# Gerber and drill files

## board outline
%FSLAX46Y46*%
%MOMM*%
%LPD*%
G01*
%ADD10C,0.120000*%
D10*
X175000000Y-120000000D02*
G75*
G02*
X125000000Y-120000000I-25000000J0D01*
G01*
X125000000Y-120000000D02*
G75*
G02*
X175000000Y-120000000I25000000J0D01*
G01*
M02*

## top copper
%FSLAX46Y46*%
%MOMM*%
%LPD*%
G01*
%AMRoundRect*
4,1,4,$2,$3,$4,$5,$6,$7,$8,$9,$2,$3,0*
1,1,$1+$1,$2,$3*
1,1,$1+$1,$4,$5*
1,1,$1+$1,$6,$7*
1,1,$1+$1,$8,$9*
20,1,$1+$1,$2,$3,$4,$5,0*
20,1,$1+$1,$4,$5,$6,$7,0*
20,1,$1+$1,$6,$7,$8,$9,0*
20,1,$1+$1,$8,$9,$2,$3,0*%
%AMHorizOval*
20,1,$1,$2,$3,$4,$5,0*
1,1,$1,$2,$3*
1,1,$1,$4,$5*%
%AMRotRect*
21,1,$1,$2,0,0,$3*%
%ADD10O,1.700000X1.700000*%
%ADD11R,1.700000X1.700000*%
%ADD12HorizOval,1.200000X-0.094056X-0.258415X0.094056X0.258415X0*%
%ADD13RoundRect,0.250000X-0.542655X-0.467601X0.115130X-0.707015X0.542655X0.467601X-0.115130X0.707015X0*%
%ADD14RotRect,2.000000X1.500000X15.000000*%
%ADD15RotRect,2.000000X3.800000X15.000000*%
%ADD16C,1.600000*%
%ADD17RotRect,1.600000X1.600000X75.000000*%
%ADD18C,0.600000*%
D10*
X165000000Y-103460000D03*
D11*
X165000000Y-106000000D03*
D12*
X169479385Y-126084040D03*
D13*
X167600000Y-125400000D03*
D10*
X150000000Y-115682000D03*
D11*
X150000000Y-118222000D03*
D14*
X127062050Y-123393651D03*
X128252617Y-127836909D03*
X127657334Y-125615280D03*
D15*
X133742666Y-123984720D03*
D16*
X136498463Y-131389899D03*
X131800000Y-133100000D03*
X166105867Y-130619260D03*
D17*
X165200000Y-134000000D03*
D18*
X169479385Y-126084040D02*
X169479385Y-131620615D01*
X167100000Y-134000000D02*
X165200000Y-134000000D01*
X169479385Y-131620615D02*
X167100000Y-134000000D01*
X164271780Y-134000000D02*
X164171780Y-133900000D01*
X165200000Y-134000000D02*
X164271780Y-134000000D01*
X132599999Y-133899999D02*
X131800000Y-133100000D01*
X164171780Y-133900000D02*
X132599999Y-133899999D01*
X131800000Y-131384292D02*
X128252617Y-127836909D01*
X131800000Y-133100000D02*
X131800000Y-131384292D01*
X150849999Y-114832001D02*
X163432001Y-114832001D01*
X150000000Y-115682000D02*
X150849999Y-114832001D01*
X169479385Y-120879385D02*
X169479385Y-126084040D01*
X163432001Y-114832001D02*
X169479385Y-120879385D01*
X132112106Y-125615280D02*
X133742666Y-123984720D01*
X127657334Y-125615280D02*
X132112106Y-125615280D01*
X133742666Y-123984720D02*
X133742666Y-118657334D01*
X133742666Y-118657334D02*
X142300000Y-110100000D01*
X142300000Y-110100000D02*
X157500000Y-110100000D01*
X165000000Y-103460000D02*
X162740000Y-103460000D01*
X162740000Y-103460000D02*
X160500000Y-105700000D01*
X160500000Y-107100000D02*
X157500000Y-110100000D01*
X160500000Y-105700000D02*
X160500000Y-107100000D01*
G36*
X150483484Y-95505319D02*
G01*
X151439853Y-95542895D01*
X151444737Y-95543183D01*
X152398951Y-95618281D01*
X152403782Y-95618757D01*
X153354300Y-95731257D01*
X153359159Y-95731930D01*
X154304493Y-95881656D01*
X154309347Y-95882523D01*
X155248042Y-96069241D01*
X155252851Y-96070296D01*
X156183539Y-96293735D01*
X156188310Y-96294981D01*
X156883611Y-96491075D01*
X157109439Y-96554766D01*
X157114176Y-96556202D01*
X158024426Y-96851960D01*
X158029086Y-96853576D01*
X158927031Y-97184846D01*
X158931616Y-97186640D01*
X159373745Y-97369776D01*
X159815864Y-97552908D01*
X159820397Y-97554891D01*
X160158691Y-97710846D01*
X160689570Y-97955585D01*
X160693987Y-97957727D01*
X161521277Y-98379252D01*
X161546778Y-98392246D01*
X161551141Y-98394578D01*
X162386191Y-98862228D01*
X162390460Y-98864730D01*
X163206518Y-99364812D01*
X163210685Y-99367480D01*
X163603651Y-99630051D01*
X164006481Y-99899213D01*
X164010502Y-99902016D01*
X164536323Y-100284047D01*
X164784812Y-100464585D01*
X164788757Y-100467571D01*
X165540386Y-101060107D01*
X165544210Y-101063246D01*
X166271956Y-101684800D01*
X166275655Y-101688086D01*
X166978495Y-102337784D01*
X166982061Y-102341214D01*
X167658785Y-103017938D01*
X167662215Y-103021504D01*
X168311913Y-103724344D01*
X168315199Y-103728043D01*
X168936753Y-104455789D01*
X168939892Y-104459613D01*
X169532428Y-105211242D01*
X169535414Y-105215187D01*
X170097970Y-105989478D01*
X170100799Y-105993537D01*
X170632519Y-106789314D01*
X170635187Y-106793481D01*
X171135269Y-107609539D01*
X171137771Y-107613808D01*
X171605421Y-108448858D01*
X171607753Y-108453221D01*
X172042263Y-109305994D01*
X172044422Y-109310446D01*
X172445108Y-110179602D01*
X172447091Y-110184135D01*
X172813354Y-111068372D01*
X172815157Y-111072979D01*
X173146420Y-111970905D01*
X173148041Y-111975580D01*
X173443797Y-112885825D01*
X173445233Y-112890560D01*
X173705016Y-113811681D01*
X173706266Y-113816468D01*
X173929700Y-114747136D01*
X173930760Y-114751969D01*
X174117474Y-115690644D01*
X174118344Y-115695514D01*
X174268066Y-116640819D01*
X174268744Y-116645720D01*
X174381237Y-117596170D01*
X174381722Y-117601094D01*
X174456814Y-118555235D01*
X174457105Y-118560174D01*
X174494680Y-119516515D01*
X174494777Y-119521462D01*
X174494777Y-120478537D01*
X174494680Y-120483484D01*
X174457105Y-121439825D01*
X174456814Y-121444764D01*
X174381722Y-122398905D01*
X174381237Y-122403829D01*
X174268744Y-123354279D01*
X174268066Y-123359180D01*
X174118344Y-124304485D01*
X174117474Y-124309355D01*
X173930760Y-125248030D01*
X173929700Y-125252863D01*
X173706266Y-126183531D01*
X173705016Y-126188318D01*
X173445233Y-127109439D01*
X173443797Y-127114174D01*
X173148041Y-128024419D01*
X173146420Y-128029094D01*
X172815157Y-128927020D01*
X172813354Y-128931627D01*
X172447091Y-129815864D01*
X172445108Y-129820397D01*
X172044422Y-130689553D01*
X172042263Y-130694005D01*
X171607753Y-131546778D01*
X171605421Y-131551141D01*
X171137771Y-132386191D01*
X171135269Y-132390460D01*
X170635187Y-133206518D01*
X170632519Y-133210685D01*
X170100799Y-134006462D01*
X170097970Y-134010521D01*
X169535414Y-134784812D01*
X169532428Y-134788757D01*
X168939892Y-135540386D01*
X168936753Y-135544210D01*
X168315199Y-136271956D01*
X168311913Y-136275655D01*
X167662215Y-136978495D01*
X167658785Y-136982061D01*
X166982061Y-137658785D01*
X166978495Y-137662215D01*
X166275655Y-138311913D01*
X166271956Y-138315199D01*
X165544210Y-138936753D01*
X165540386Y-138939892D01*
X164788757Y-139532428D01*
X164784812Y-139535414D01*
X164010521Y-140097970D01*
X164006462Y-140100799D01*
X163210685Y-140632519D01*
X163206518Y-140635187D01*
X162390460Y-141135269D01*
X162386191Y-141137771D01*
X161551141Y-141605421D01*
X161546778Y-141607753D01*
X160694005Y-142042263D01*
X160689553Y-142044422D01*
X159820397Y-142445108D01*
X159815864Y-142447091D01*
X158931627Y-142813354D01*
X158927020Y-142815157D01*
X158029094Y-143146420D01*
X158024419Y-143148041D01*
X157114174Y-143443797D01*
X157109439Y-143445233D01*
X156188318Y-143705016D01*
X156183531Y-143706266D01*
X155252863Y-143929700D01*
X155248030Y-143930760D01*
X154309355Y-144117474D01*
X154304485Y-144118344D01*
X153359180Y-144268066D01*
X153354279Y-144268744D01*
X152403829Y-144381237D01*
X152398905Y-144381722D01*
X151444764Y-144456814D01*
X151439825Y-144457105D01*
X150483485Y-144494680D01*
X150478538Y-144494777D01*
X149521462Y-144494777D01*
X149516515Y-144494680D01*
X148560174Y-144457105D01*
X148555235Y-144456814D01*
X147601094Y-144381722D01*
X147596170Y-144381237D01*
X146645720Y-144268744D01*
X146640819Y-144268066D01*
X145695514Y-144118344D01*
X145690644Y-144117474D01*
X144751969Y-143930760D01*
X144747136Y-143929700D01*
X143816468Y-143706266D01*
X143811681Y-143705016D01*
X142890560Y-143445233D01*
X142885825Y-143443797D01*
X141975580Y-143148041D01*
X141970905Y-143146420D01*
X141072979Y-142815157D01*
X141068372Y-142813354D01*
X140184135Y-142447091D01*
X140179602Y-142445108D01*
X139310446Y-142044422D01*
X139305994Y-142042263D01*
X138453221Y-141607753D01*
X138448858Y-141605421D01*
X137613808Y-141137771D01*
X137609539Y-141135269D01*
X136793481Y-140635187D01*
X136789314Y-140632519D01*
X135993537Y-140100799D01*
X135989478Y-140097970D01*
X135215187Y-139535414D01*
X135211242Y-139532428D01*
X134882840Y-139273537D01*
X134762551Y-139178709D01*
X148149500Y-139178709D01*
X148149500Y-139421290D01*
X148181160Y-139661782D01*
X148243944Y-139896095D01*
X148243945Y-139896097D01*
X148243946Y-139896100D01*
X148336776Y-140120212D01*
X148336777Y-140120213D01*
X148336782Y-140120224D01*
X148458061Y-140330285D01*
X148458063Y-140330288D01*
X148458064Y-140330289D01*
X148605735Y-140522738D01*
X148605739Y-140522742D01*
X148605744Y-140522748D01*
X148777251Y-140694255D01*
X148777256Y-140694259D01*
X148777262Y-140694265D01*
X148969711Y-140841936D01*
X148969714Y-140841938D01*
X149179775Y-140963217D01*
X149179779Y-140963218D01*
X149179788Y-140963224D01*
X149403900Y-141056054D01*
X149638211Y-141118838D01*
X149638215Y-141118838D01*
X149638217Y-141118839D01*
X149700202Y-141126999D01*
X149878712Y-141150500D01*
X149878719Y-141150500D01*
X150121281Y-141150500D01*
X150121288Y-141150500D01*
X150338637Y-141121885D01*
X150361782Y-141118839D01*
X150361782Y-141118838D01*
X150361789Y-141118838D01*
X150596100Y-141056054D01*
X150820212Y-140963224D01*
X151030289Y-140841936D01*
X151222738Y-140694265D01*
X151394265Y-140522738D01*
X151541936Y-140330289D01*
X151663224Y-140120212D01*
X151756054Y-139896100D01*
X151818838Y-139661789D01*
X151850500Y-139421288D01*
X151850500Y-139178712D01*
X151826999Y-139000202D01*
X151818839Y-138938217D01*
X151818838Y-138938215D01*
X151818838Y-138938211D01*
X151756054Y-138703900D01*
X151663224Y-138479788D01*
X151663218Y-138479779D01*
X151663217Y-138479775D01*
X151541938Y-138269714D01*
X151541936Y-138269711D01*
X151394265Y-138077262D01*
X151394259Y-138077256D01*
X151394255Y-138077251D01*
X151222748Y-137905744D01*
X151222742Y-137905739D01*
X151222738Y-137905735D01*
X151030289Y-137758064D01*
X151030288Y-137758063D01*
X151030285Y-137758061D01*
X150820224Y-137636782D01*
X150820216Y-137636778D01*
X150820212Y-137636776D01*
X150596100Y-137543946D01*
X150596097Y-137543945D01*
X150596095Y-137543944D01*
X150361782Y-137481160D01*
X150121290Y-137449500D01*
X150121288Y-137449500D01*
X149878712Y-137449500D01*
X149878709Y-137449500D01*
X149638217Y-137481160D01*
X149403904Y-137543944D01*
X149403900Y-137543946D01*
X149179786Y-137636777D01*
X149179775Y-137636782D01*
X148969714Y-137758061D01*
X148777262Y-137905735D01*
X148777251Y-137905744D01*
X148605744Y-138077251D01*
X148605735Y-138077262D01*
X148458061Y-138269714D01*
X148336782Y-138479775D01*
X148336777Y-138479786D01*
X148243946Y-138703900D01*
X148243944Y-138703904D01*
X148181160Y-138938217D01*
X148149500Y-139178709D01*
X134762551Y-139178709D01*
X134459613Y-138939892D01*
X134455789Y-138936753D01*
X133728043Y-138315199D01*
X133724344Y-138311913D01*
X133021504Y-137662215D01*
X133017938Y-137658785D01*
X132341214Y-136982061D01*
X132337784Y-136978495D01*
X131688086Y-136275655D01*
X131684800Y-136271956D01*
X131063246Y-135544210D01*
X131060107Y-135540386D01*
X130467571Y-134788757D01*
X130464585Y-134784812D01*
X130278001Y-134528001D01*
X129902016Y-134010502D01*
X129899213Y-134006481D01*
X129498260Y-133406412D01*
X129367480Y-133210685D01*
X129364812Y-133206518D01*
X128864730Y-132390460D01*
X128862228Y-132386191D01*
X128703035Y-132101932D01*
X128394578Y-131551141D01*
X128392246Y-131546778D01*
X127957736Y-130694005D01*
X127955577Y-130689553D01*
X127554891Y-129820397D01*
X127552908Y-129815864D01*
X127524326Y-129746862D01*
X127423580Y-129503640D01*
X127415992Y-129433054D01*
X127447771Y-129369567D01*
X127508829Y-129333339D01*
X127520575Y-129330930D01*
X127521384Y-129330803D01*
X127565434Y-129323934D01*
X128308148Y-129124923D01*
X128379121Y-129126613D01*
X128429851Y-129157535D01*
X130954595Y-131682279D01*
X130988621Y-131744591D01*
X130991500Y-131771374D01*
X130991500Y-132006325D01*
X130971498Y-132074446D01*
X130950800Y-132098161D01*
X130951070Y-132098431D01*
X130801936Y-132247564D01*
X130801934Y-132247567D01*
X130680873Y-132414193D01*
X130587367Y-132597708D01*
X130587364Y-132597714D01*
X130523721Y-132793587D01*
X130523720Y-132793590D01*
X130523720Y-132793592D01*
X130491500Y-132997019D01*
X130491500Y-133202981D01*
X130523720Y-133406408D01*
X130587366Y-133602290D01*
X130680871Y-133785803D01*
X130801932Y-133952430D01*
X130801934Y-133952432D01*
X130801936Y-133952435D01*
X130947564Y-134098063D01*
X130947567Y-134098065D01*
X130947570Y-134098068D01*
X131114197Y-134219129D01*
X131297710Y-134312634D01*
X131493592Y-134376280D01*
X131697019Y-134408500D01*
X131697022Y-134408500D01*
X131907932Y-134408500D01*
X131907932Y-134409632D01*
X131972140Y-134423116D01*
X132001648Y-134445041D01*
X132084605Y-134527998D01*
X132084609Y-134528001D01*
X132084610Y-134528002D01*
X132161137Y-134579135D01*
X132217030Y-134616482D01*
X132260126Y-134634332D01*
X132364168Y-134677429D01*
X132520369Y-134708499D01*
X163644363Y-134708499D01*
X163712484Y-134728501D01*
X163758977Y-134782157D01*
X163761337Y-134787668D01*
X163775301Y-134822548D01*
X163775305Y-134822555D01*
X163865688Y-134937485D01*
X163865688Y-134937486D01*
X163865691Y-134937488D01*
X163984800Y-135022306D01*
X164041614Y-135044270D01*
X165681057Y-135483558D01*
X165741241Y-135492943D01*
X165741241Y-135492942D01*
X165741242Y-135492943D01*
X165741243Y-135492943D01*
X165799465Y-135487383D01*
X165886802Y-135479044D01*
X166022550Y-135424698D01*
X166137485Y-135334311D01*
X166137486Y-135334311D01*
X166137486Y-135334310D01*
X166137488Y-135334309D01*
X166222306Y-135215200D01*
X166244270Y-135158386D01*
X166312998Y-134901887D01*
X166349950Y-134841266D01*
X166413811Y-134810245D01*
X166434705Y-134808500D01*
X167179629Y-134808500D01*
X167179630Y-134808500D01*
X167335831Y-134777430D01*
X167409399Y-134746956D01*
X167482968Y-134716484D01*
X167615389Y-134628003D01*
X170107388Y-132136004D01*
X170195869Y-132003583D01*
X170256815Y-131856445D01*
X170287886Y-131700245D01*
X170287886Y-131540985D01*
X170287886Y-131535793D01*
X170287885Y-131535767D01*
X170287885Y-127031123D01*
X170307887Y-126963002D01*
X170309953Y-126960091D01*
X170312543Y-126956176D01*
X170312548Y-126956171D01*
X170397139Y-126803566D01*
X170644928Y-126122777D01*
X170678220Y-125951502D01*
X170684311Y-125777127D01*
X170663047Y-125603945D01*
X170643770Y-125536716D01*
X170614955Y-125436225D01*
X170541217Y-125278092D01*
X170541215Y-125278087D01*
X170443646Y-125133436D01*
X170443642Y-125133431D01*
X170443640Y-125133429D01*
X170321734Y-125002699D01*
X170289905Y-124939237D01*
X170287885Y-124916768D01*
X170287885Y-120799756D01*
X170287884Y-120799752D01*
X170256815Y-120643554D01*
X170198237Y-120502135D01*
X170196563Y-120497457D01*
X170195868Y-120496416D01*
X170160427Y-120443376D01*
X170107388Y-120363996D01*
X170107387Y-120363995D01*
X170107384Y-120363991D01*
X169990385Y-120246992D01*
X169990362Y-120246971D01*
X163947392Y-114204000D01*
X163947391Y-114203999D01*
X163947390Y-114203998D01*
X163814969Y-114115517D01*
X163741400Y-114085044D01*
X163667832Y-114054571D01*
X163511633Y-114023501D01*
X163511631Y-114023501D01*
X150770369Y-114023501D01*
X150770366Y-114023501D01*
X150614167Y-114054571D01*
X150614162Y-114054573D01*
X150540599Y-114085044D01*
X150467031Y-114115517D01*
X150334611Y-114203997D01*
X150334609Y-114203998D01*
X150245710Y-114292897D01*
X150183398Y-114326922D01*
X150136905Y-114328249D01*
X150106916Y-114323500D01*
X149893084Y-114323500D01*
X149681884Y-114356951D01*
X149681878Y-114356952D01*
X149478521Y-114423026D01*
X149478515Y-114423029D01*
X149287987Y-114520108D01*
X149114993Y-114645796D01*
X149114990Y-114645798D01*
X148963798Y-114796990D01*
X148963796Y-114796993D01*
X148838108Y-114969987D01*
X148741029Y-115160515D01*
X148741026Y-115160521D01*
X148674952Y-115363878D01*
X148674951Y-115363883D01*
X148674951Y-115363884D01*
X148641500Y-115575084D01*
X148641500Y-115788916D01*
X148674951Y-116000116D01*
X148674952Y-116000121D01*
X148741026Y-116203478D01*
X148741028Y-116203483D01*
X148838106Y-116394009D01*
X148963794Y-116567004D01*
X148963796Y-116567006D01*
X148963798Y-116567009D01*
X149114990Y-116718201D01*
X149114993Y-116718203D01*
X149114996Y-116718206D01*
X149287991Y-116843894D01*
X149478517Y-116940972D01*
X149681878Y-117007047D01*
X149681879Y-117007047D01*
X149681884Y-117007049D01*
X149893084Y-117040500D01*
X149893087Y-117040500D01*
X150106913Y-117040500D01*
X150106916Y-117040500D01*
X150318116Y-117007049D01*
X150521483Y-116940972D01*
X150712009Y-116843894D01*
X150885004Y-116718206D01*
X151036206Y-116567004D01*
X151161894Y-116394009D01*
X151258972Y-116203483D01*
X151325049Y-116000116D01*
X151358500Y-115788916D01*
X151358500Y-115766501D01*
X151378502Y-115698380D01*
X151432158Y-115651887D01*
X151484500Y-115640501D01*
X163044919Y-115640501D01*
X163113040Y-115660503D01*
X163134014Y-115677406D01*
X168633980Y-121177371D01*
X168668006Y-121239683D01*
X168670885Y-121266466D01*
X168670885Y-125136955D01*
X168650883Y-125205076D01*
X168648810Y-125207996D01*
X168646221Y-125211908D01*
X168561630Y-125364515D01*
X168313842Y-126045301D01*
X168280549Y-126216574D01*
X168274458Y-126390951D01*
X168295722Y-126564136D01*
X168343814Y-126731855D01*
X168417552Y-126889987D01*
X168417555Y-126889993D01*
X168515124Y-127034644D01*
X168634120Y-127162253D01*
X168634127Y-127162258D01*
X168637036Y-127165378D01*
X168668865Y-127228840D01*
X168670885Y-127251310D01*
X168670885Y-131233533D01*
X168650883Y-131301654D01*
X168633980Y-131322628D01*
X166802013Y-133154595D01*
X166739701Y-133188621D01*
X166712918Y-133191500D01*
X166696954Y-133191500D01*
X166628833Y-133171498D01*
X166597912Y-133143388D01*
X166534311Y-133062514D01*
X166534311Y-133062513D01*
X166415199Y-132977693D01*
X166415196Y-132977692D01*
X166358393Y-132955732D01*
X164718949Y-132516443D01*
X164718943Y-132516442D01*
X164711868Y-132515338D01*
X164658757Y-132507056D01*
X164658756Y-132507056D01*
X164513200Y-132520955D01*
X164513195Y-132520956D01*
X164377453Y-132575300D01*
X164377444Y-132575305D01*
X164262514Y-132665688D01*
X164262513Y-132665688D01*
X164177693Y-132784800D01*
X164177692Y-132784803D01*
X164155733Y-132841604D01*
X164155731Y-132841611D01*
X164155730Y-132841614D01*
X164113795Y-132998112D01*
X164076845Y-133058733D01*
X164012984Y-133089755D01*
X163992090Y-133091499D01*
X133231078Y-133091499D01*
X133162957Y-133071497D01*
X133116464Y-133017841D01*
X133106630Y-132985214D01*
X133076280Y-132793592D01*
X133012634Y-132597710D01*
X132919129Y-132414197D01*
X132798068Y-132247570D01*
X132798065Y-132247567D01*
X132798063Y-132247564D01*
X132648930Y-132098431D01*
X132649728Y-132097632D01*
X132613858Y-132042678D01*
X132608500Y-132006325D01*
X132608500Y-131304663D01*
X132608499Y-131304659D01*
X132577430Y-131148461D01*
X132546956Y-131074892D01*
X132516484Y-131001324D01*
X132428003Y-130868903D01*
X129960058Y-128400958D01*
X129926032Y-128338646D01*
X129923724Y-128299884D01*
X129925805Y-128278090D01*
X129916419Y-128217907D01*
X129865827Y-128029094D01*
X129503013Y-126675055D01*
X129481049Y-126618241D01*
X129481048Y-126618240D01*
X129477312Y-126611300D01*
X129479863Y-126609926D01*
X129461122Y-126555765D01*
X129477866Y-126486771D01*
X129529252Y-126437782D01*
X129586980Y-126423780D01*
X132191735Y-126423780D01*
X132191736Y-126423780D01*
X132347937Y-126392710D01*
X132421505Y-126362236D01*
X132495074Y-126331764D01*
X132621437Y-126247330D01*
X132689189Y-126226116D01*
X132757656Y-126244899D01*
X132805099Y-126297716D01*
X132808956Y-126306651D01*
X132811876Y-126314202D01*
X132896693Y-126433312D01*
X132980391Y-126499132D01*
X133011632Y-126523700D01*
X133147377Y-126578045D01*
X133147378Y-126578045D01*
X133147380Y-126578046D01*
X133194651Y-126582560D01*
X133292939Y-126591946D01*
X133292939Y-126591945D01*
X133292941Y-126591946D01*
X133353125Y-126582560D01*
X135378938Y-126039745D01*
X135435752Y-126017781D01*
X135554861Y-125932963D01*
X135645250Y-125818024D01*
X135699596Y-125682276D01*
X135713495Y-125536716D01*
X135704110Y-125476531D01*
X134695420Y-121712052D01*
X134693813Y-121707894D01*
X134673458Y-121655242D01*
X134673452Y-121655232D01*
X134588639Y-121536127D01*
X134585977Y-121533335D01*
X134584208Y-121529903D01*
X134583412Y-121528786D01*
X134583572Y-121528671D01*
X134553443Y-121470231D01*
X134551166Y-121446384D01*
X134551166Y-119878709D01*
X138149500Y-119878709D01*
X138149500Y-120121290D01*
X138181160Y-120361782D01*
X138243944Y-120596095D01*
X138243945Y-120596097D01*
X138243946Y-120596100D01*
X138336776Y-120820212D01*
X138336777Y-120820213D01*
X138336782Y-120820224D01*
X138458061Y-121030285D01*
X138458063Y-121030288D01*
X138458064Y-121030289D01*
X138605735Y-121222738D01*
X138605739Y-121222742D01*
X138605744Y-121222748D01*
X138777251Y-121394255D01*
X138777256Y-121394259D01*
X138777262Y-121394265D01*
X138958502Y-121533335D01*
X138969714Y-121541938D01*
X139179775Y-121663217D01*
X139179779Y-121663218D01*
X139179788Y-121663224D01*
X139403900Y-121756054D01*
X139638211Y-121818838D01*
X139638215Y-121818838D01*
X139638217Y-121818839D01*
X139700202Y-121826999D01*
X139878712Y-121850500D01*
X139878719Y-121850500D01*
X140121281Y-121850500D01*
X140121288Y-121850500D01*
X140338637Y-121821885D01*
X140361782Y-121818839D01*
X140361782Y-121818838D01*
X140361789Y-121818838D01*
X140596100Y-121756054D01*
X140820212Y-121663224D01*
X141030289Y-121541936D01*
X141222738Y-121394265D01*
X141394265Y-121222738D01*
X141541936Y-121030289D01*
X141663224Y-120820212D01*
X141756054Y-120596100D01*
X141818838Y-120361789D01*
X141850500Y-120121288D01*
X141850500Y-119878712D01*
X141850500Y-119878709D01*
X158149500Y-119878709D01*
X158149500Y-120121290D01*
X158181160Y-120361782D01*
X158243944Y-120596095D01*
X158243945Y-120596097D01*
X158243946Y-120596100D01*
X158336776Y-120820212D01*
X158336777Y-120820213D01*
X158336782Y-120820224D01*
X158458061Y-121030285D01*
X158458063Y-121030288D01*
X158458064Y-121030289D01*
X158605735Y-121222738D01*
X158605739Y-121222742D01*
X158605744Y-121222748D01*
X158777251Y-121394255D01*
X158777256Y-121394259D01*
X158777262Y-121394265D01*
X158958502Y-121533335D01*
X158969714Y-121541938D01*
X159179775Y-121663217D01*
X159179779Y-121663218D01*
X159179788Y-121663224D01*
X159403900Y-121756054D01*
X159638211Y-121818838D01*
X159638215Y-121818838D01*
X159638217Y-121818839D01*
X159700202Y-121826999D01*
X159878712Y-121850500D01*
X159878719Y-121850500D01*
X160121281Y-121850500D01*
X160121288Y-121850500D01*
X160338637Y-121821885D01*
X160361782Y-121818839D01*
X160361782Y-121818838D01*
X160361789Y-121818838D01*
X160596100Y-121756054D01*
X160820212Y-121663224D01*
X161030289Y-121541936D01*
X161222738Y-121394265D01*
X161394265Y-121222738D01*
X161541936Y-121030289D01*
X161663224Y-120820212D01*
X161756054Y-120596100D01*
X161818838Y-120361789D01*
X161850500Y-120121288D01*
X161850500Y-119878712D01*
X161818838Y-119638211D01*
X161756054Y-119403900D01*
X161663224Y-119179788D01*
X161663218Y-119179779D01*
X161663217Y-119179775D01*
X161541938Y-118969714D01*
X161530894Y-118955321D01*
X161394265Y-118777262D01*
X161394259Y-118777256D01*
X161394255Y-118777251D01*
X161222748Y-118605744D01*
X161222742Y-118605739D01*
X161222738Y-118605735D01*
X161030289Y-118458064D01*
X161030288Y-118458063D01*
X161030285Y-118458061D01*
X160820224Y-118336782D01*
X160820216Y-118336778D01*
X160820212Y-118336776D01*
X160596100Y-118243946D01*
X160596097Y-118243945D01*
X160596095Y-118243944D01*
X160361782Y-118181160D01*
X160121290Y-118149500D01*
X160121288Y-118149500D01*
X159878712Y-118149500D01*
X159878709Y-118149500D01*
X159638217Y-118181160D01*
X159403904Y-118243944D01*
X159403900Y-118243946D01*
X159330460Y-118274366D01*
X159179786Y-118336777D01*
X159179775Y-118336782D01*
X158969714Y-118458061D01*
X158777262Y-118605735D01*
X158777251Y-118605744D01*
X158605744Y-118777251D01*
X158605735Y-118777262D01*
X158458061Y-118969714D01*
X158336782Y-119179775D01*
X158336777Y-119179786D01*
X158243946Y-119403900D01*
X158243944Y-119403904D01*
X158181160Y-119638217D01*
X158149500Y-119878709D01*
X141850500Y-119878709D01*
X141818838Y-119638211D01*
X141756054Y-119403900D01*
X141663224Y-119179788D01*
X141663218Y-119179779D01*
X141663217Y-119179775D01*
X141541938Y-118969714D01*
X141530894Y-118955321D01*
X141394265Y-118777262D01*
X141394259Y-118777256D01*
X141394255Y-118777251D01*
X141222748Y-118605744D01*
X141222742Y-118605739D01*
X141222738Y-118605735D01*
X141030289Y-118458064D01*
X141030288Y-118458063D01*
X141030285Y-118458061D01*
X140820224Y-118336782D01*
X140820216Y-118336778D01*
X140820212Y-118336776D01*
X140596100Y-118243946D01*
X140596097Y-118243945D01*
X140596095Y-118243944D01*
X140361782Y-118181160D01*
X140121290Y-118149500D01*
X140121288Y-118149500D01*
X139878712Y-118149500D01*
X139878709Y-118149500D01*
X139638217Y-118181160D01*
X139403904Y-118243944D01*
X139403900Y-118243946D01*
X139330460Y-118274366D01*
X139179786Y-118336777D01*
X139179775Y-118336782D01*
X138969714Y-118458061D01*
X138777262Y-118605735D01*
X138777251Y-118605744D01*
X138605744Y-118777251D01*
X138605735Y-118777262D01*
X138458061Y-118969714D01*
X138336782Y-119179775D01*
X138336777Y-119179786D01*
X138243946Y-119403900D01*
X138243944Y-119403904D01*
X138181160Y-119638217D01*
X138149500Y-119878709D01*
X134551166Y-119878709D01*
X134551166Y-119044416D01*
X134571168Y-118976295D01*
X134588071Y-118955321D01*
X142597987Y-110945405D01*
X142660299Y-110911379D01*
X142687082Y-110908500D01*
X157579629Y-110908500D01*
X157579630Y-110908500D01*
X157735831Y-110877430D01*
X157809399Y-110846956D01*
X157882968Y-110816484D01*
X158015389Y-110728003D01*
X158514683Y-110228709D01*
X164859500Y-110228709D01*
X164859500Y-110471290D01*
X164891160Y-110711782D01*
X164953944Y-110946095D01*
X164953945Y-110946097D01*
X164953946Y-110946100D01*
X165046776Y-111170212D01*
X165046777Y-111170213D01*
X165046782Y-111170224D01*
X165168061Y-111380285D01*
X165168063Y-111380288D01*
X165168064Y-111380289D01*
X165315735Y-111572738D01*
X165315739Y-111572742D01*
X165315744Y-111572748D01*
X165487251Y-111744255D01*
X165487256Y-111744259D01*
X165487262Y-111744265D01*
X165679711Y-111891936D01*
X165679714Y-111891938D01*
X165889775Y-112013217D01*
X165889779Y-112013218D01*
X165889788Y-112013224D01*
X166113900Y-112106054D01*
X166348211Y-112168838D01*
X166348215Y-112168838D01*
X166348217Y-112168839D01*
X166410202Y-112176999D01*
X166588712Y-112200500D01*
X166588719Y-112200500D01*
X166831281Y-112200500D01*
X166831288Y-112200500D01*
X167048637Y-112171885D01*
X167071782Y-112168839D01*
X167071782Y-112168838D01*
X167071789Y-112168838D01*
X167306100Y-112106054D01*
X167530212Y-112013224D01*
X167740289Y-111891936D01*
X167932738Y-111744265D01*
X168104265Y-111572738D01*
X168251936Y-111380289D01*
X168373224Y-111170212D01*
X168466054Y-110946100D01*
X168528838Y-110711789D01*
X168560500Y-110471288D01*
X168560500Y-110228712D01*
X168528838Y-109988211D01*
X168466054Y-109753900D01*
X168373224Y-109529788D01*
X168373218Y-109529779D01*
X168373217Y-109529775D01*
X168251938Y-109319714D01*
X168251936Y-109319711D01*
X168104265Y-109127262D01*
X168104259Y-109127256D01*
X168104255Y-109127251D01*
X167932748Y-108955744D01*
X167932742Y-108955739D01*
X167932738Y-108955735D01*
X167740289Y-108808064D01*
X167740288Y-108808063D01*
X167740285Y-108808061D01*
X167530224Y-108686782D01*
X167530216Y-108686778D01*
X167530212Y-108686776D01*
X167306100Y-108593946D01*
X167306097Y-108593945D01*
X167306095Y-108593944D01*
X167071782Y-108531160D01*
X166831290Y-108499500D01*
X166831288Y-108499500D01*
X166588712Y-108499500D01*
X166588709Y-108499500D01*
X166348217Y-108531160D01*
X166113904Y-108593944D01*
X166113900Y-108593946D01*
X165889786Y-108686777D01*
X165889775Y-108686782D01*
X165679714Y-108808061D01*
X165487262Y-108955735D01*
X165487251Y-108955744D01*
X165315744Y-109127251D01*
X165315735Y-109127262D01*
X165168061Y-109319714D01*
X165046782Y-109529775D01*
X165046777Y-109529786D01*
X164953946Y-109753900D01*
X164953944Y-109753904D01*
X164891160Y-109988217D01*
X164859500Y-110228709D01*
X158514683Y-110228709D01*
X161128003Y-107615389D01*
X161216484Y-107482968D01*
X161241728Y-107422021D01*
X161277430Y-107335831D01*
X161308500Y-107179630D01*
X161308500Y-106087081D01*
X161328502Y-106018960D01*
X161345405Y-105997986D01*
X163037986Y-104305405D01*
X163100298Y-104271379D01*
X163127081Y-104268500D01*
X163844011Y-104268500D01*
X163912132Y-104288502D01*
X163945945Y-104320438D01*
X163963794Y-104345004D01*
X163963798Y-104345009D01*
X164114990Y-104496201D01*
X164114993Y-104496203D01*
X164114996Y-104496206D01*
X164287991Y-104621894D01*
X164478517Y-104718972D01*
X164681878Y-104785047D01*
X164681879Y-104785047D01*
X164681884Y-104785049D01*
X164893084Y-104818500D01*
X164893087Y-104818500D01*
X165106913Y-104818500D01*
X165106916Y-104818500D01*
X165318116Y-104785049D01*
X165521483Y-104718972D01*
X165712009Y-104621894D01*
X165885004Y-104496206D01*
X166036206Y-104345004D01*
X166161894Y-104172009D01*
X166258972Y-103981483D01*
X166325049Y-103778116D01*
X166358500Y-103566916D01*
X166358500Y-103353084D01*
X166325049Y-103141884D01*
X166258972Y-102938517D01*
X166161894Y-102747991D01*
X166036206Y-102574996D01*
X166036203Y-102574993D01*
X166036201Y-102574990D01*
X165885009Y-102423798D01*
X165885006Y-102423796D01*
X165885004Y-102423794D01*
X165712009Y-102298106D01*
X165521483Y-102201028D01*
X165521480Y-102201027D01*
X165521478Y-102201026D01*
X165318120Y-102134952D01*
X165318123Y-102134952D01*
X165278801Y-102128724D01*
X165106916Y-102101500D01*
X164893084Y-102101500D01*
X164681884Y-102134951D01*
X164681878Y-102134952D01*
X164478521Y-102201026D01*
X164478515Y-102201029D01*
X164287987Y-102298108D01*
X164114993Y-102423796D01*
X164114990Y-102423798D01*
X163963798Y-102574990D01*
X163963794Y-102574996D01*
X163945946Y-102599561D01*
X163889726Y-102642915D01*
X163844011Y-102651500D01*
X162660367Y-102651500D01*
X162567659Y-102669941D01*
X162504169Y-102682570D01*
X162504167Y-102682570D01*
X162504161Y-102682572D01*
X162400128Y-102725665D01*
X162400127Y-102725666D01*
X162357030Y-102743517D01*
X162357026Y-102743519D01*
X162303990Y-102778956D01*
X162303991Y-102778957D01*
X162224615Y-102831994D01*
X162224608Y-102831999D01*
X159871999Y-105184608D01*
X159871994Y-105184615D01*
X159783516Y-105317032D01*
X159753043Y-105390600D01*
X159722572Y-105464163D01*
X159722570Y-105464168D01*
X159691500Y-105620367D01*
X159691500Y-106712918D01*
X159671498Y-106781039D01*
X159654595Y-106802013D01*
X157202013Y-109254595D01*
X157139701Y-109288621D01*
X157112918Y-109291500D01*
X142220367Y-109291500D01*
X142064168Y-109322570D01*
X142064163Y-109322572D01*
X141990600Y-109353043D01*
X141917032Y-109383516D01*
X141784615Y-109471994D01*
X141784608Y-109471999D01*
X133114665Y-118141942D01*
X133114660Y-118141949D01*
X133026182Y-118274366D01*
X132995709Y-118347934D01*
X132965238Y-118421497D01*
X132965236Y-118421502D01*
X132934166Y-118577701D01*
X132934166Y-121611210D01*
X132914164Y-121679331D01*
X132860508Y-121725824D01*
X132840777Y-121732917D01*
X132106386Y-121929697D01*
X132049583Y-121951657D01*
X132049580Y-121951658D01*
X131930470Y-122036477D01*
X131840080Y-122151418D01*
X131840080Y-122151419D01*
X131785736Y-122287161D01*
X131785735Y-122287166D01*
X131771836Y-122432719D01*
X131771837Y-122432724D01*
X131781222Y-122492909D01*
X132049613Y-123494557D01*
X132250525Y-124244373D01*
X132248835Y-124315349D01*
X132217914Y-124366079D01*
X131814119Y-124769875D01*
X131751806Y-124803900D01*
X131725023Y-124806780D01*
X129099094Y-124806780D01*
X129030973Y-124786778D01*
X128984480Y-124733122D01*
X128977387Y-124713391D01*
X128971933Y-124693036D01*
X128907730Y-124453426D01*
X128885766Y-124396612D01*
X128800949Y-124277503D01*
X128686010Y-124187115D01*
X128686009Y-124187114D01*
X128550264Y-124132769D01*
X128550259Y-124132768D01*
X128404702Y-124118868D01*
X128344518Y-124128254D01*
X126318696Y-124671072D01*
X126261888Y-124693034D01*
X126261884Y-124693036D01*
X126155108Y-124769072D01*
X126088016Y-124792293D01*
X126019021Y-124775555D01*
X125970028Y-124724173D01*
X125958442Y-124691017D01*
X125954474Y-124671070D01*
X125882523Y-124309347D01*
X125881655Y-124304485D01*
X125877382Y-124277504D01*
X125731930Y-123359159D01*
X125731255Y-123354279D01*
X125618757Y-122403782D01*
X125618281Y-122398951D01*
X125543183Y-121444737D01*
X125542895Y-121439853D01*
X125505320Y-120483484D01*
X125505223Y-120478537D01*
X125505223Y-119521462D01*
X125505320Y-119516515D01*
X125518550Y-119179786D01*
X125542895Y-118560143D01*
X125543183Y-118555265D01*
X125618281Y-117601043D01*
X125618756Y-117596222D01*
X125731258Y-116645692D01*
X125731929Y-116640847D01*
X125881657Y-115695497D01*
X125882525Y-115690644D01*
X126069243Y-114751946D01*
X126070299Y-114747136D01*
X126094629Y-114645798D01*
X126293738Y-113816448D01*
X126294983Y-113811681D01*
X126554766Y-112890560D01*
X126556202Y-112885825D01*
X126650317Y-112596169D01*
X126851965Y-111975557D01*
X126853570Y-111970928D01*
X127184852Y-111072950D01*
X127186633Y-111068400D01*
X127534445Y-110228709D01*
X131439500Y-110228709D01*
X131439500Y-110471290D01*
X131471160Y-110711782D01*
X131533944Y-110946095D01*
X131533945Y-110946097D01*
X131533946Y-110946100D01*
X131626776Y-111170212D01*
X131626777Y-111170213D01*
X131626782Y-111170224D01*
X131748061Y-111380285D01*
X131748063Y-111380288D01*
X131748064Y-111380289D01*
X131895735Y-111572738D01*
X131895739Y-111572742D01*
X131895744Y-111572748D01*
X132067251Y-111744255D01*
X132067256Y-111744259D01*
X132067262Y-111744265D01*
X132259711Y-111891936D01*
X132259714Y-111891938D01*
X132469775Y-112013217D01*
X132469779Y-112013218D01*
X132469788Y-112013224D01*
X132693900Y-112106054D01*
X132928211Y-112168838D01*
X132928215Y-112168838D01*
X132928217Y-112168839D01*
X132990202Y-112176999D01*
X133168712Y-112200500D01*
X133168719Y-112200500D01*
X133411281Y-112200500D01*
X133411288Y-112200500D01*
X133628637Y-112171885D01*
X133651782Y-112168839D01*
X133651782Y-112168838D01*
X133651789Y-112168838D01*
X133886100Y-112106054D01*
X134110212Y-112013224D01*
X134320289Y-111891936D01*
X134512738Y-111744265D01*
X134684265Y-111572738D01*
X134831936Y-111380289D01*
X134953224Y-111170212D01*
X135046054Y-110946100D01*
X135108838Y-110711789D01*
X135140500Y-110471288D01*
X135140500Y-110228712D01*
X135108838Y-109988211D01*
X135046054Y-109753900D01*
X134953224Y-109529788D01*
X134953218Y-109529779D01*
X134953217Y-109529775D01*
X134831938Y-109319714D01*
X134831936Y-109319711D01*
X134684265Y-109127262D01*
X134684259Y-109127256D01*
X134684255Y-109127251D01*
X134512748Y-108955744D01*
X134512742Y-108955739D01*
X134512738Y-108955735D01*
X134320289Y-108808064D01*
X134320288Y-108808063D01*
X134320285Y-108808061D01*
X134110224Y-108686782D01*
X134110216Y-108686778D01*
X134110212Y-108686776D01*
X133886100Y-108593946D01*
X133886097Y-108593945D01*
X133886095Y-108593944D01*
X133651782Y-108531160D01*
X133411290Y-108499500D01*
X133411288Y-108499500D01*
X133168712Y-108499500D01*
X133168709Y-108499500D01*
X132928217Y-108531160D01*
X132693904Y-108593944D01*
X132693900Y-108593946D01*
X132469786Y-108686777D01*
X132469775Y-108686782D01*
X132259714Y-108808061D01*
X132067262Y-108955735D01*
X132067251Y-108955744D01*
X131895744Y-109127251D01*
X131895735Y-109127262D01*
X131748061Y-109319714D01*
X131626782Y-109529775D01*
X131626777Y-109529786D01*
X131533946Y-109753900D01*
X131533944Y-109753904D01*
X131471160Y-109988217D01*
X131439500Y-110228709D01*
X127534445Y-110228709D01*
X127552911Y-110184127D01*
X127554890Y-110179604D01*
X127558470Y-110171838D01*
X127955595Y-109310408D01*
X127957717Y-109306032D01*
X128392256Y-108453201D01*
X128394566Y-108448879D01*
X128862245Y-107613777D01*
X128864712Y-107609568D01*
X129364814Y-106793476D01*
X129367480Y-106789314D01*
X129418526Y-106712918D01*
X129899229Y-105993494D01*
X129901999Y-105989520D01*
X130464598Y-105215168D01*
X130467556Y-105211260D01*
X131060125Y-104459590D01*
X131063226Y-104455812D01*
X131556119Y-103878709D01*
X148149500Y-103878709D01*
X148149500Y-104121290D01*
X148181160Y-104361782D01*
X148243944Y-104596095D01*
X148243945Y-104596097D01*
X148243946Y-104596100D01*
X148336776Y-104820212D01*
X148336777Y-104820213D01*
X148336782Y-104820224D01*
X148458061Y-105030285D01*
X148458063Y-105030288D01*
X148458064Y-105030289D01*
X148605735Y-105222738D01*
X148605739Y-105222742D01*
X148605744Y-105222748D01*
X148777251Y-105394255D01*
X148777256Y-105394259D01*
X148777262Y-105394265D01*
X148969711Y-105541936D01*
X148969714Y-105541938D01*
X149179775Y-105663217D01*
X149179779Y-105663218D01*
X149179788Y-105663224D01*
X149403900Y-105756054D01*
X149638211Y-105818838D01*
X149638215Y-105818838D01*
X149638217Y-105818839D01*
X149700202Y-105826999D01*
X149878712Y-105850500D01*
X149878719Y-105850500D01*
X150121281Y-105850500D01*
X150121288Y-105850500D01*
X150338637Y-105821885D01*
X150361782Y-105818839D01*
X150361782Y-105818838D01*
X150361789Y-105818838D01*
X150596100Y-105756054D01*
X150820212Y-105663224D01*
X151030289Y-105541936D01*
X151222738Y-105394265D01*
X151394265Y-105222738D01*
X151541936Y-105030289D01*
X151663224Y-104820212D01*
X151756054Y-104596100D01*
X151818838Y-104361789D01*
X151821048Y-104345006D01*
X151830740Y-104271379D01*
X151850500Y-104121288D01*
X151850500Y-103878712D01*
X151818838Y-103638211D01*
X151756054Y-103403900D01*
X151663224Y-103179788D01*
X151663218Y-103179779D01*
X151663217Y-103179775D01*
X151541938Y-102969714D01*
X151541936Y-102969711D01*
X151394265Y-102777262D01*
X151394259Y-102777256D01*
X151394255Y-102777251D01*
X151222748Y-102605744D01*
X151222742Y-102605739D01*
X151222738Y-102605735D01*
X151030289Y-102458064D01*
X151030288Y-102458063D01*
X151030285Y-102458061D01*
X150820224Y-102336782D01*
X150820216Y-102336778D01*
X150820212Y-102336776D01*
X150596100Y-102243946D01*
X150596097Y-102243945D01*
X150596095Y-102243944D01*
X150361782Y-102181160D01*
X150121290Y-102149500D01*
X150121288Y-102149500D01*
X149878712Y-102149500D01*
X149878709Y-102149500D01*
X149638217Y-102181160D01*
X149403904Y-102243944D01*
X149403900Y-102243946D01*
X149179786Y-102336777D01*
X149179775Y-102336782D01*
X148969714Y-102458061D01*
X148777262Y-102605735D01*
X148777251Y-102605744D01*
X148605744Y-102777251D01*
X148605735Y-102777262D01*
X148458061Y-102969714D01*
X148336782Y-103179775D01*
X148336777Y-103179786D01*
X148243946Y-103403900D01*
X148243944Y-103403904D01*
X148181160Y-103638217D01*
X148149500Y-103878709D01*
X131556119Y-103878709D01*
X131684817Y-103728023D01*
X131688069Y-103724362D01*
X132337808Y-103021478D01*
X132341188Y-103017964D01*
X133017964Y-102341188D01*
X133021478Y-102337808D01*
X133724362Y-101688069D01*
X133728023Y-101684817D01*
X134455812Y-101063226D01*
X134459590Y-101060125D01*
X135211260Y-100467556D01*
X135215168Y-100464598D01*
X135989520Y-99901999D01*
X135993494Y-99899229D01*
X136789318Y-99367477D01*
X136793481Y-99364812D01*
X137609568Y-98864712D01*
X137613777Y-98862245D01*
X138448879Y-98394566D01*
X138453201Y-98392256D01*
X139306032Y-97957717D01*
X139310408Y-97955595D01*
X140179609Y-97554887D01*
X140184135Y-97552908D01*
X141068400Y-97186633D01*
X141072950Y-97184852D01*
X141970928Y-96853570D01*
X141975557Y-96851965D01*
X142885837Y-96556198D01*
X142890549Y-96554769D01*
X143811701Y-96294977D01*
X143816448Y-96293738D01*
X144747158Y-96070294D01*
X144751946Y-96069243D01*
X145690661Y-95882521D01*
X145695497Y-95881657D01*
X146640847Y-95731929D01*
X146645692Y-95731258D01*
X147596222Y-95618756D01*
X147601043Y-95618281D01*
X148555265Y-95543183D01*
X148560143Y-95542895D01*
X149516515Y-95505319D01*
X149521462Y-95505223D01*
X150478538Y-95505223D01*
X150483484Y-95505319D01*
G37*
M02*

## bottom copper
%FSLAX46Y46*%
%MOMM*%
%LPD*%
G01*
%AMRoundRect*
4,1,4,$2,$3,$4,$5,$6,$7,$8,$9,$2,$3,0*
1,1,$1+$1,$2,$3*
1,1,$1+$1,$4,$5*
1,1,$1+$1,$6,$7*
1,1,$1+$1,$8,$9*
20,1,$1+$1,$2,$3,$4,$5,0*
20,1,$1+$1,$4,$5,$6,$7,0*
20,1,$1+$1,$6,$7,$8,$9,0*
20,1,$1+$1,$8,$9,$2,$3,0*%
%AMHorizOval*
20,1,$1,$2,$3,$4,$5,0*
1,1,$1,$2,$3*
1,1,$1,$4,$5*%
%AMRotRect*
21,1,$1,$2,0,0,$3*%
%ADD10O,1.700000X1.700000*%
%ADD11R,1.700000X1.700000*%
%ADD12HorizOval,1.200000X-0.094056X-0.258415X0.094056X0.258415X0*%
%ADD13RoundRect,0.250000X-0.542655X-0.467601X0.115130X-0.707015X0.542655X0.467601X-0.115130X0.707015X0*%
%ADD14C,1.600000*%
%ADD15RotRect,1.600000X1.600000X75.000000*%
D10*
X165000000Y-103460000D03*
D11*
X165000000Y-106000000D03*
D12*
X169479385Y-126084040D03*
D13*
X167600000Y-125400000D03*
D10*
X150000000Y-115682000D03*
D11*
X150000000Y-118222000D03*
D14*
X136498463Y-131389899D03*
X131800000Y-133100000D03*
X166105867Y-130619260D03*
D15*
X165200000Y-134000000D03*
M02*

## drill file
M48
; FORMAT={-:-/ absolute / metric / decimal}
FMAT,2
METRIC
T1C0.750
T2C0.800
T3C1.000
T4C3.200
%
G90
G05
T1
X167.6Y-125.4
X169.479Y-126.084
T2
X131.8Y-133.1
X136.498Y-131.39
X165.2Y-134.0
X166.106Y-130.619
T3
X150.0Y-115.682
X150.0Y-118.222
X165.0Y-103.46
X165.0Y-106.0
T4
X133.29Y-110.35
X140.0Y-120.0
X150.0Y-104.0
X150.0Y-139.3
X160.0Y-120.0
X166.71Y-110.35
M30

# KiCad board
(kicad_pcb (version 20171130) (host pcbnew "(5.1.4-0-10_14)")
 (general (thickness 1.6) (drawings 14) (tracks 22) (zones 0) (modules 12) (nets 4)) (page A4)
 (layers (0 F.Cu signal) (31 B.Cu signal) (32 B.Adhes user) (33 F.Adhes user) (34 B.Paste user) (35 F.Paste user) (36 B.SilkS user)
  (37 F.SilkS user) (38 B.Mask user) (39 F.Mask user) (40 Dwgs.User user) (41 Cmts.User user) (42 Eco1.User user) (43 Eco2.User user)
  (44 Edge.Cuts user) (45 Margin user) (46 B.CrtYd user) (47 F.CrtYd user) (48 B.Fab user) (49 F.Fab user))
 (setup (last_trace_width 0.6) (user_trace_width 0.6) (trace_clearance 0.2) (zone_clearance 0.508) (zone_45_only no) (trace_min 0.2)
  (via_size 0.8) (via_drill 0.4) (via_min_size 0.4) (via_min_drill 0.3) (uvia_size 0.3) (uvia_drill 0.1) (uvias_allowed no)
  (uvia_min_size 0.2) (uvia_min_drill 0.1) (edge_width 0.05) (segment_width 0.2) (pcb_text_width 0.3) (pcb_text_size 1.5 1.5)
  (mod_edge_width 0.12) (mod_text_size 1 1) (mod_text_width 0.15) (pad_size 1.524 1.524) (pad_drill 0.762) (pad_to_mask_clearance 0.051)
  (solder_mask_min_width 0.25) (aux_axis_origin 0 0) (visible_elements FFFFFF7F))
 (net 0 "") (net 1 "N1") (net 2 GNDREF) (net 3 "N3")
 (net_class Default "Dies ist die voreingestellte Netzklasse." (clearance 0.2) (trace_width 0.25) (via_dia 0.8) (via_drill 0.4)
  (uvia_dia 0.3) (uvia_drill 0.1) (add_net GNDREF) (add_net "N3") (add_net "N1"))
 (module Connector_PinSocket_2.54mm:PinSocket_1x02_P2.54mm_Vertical (layer B.Cu) (at 165 106)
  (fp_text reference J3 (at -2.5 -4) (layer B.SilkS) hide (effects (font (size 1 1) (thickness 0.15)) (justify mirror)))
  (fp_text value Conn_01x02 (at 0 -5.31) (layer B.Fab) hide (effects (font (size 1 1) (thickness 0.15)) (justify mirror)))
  (pad 2 thru_hole oval (at 0 -2.54) (size 1.7 1.7) (drill 1) (layers *.Cu *.Mask) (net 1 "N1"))
  (pad 1 thru_hole rect (at 0 0) (size 1.7 1.7) (drill 1) (layers *.Cu *.Mask) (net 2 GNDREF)))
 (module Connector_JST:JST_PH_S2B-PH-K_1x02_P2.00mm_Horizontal (layer B.Cu) (at 167.6 125.4 340)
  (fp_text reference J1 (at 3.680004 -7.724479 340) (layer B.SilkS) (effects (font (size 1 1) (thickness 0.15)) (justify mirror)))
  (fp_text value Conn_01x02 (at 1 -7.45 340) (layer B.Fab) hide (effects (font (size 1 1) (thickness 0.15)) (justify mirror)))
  (pad 2 thru_hole oval (at 2 0 340) (size 1.2 1.75) (drill 0.75) (layers *.Cu *.Mask) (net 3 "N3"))
  (pad 1 thru_hole roundrect (at 0 0 340) (size 1.2 1.75) (drill 0.75) (layers *.Cu *.Mask) (roundrect_rratio 0.208333) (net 2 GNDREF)))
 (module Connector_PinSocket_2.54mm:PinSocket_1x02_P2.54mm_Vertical (layer F.Cu) (at 150 118.222 180)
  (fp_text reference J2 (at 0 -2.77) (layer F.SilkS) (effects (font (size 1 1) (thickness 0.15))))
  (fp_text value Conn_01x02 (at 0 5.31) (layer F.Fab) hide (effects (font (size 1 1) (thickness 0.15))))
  (pad 2 thru_hole oval (at 0 2.54 180) (size 1.7 1.7) (drill 1) (layers *.Cu *.Mask) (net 3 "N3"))
  (pad 1 thru_hole rect (at 0 0 180) (size 1.7 1.7) (drill 1) (layers *.Cu *.Mask) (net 2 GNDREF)))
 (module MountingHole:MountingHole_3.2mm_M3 (layer F.Cu) (at 160 120)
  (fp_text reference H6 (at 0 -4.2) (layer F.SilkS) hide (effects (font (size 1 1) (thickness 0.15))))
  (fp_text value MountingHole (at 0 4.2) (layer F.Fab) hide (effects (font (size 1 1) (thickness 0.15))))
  (pad 1 np_thru_hole circle (at 0 0) (size 3.2 3.2) (drill 3.2) (layers *.Cu *.Mask)))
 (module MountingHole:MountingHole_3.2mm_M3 (layer F.Cu) (at 140 120)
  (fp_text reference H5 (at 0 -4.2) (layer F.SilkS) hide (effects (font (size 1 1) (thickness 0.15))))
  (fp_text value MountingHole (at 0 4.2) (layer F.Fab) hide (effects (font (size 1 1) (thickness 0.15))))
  (pad 1 np_thru_hole circle (at 0 0) (size 3.2 3.2) (drill 3.2) (layers *.Cu *.Mask)))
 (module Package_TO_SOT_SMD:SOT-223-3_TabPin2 (layer F.Cu) (at 130.7 124.8 15)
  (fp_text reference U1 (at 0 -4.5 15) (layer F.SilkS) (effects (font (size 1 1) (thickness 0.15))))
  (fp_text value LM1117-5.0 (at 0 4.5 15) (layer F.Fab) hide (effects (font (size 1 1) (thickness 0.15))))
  (pad 1 smd rect (at -3.15 -2.3 15) (size 2 1.5) (layers F.Cu F.Paste F.Mask) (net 2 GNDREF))
  (pad 3 smd rect (at -3.15 2.3 15) (size 2 1.5) (layers F.Cu F.Paste F.Mask) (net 3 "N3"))
  (pad 2 smd rect (at -3.15 0 15) (size 2 1.5) (layers F.Cu F.Paste F.Mask) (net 1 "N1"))
  (pad 2 smd rect (at 3.15 0 15) (size 2 3.8) (layers F.Cu F.Paste F.Mask) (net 1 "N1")))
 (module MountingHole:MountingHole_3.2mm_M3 (layer F.Cu) (at 133.29 110.35)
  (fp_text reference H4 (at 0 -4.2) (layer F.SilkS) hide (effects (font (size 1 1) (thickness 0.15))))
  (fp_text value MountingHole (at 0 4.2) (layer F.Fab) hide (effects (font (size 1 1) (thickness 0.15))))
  (pad 1 np_thru_hole circle (at 0 0) (size 3.2 3.2) (drill 3.2) (layers *.Cu *.Mask)))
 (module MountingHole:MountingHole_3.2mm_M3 (layer F.Cu) (at 166.71 110.35)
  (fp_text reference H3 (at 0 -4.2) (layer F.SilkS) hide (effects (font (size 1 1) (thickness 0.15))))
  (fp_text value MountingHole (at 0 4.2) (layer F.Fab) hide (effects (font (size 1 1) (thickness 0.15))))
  (pad 1 np_thru_hole circle (at 0 0) (size 3.2 3.2) (drill 3.2) (layers *.Cu *.Mask)))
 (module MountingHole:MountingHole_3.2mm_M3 (layer F.Cu) (at 150 139.3)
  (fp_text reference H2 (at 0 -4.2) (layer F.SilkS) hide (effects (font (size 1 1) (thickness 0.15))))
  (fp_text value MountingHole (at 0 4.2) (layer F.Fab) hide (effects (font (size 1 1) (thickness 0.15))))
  (pad 1 np_thru_hole circle (at 0 0) (size 3.2 3.2) (drill 3.2) (layers *.Cu *.Mask)))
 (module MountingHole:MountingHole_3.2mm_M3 (layer F.Cu) (at 150 104)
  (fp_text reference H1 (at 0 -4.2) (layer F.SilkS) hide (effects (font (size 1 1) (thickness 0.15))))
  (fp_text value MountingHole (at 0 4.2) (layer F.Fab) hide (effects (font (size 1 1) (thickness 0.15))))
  (pad 1 np_thru_hole circle (at 0 0) (size 3.2 3.2) (drill 3.2) (layers *.Cu *.Mask)))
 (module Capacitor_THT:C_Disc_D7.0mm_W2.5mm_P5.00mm (layer F.Cu) (at 131.8 133.1 20)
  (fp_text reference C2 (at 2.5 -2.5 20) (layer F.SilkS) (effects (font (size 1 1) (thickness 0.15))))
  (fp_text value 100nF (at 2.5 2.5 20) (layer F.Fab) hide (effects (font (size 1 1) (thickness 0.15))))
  (pad 2 thru_hole circle (at 5 0 20) (size 1.6 1.6) (drill 0.8) (layers *.Cu *.Mask) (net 2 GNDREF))
  (pad 1 thru_hole circle (at 0 0 20) (size 1.6 1.6) (drill 0.8) (layers *.Cu *.Mask) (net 3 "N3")))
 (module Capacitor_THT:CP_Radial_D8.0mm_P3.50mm (layer F.Cu) (at 165.2 134 75)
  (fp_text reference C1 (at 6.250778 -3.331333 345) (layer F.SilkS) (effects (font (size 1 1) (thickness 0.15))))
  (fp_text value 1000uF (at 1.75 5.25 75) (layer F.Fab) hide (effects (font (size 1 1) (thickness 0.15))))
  (pad 2 thru_hole circle (at 3.5 0 75) (size 1.6 1.6) (drill 0.8) (layers *.Cu *.Mask) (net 2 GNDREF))
  (pad 1 thru_hole rect (at 0 0 75) (size 1.6 1.6) (drill 0.8) (layers *.Cu *.Mask) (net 3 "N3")))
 (gr_circle (center 150 120) (end 175 120) (layer Edge.Cuts) (width 0.12))
 (segment (start 169.479385 126.08404) (end 169.479385 131.620615) (width 0.6) (layer F.Cu) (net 3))
 (segment (start 167.1 134) (end 165.2 134) (width 0.6) (layer F.Cu) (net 3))
 (segment (start 169.479385 131.620615) (end 167.1 134) (width 0.6) (layer F.Cu) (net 3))
 (segment (start 164.27178 134) (end 164.17178 133.9) (width 0.6) (layer F.Cu) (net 3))
 (segment (start 165.2 134) (end 164.27178 134) (width 0.6) (layer F.Cu) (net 3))
 (segment (start 132.599999 133.899999) (end 131.8 133.1) (width 0.6) (layer F.Cu) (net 3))
 (segment (start 164.17178 133.9) (end 132.599999 133.899999) (width 0.6) (layer F.Cu) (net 3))
 (segment (start 131.8 131.384292) (end 128.252617 127.836909) (width 0.6) (layer F.Cu) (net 3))
 (segment (start 131.8 133.1) (end 131.8 131.384292) (width 0.6) (layer F.Cu) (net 3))
 (segment (start 150.849999 114.832001) (end 163.432001 114.832001) (width 0.6) (layer F.Cu) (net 3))
 (segment (start 150 115.682) (end 150.849999 114.832001) (width 0.6) (layer F.Cu) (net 3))
 (segment (start 169.479385 120.879385) (end 169.479385 126.08404) (width 0.6) (layer F.Cu) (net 3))
 (segment (start 163.432001 114.832001) (end 169.479385 120.879385) (width 0.6) (layer F.Cu) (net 3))
 (segment (start 132.112106 125.61528) (end 133.742666 123.98472) (width 0.6) (layer F.Cu) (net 1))
 (segment (start 127.657334 125.61528) (end 132.112106 125.61528) (width 0.6) (layer F.Cu) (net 1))
 (segment (start 133.742666 123.98472) (end 133.742666 118.657334) (width 0.6) (layer F.Cu) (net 1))
 (segment (start 133.742666 118.657334) (end 142.3 110.1) (width 0.6) (layer F.Cu) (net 1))
 (segment (start 142.3 110.1) (end 157.5 110.1) (width 0.6) (layer F.Cu) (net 1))
 (segment (start 165 103.46) (end 162.74 103.46) (width 0.6) (layer F.Cu) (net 1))
 (segment (start 162.74 103.46) (end 160.5 105.7) (width 0.6) (layer F.Cu) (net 1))
 (segment (start 160.5 107.1) (end 157.5 110.1) (width 0.6) (layer F.Cu) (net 1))
 (segment (start 160.5 105.7) (end 160.5 107.1) (width 0.6) (layer F.Cu) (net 1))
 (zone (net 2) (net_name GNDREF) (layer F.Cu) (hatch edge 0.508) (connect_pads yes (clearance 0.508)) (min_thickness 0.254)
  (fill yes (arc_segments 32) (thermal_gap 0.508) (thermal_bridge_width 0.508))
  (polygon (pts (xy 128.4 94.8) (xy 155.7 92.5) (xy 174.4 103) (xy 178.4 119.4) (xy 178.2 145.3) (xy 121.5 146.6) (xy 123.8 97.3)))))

